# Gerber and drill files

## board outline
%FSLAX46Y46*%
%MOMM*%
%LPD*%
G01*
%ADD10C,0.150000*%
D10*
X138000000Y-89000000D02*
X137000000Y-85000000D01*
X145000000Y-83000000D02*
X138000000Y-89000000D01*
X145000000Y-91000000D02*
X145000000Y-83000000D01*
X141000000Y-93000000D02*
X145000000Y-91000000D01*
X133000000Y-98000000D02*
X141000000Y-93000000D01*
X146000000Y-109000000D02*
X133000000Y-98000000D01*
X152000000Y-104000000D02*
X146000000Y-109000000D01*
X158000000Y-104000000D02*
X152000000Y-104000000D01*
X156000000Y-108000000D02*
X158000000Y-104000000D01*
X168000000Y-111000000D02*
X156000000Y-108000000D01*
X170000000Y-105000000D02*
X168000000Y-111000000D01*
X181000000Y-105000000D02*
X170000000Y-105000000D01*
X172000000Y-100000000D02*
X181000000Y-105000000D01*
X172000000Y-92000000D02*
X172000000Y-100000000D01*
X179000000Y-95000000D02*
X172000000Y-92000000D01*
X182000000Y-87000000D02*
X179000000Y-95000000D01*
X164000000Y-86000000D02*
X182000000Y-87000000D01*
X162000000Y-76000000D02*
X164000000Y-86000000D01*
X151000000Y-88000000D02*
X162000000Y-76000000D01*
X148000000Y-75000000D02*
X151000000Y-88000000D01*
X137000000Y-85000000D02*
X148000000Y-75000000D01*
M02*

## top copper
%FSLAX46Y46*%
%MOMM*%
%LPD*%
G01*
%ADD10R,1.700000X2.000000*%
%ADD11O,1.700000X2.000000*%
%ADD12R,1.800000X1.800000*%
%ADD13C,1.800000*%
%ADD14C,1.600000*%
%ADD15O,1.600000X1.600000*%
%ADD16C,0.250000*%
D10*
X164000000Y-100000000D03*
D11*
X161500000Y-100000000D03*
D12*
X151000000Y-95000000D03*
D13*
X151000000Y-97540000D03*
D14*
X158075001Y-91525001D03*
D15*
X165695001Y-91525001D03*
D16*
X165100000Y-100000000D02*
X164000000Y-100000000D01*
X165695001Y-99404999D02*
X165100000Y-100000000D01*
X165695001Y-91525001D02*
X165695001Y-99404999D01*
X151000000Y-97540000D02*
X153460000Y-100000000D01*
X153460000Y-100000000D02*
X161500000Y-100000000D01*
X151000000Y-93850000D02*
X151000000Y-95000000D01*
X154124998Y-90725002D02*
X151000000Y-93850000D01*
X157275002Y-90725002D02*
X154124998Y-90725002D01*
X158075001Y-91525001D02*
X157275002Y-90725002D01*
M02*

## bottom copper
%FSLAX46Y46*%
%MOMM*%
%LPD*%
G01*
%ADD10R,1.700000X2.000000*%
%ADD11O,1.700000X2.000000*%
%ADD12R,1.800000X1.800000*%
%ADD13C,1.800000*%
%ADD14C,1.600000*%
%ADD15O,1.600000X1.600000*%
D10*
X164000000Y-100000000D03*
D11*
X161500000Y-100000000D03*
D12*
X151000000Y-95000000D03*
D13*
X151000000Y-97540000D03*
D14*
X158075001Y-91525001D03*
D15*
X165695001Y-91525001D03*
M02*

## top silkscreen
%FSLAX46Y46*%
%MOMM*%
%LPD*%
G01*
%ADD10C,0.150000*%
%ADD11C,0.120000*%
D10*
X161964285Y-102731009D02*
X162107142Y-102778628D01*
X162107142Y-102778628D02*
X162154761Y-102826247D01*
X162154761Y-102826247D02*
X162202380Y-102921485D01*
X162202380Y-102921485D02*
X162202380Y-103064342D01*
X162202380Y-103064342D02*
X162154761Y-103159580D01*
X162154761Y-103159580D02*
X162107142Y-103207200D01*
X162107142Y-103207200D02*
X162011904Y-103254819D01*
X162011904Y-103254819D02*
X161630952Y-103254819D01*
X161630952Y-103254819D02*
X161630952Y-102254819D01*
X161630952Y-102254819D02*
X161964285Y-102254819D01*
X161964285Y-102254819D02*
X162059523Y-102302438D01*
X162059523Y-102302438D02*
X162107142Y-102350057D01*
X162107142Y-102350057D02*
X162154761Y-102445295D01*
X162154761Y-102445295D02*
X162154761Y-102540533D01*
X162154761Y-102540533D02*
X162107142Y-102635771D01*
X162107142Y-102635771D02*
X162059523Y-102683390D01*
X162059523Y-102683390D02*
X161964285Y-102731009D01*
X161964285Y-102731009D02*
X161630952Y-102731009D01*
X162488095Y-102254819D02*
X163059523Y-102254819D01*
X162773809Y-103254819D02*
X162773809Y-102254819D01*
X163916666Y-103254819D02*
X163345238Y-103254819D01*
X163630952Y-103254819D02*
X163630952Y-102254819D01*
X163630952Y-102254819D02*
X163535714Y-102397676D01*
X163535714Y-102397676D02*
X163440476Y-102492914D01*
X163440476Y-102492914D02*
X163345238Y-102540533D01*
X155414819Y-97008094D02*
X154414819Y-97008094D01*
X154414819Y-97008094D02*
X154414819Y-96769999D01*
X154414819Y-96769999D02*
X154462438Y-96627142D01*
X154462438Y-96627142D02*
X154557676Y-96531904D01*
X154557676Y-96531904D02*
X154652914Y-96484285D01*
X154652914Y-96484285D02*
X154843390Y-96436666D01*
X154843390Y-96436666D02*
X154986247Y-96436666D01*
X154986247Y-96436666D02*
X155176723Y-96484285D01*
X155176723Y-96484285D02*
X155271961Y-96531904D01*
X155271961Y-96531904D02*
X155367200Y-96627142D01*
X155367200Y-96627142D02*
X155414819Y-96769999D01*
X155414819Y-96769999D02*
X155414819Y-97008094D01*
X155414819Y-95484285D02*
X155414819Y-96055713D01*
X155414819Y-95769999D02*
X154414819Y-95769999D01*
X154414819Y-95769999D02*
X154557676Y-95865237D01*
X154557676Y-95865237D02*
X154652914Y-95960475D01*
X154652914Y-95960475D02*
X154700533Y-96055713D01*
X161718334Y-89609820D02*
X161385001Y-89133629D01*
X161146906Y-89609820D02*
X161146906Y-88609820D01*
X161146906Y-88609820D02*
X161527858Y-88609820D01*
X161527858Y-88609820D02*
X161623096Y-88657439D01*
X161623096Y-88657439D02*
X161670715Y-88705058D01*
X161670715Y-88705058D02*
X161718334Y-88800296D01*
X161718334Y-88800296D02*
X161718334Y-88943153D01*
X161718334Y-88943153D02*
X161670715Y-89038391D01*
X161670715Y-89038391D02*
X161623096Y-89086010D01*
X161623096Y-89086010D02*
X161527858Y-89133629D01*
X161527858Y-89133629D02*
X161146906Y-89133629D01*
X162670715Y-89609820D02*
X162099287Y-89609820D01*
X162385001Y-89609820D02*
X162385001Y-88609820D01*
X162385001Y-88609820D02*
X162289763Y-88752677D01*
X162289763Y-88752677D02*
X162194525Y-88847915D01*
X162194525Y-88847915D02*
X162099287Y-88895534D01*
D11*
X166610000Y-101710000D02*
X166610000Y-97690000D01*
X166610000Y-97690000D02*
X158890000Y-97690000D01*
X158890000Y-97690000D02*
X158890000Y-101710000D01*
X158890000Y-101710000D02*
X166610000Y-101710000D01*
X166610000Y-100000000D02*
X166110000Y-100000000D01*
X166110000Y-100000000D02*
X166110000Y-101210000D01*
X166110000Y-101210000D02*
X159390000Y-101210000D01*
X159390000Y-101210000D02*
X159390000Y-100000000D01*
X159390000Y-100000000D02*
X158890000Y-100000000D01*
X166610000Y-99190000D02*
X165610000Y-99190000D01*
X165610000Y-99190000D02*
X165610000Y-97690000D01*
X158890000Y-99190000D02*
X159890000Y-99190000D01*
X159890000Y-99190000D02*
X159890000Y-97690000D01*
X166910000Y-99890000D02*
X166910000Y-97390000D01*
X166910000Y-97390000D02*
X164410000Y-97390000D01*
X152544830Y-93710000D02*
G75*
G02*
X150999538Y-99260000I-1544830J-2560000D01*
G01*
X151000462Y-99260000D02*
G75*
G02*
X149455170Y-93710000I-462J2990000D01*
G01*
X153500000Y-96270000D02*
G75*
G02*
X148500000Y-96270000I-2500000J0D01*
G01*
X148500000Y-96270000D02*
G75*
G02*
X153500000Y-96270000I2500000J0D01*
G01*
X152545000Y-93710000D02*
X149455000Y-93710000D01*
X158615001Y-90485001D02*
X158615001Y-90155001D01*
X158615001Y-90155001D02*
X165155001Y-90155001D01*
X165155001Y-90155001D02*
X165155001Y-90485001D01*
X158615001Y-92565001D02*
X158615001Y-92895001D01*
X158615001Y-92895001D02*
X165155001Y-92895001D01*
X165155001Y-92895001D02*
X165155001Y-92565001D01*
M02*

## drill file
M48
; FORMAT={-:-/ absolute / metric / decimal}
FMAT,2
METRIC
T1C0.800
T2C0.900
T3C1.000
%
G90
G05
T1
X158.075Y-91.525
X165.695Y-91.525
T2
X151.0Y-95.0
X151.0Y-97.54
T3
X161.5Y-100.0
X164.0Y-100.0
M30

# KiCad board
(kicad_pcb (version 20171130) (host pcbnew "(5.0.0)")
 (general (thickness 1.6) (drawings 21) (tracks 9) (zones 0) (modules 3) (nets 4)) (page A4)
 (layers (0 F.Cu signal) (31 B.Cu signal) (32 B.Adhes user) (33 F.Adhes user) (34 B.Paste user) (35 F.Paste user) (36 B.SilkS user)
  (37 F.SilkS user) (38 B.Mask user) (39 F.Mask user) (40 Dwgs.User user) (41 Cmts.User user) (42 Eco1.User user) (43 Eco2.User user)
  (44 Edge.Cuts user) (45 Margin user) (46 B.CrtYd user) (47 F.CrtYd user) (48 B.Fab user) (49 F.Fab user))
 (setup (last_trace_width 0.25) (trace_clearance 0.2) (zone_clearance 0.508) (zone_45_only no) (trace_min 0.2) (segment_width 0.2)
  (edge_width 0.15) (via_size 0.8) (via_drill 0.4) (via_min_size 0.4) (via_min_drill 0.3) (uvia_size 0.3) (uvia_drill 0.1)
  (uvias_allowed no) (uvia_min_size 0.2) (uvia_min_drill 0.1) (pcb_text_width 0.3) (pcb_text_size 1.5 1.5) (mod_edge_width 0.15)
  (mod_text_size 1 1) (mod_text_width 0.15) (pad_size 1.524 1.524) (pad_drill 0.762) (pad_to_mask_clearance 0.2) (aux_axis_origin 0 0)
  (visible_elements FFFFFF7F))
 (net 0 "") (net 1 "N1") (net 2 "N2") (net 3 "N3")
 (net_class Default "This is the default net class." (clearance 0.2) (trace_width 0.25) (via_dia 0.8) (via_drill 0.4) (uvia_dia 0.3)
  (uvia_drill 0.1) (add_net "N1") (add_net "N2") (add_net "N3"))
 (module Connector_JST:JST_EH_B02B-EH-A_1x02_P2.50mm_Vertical (layer F.Cu) (at 164 100 180)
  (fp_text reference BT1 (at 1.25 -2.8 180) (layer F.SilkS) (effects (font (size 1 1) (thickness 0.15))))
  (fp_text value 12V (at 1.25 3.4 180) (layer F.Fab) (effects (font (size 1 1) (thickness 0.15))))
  (fp_line (start -2.61 -1.71) (end -2.61 2.31) (layer F.SilkS) (width 0.12))
  (fp_line (start -2.61 2.31) (end 5.11 2.31) (layer F.SilkS) (width 0.12))
  (fp_line (start 5.11 2.31) (end 5.11 -1.71) (layer F.SilkS) (width 0.12))
  (fp_line (start 5.11 -1.71) (end -2.61 -1.71) (layer F.SilkS) (width 0.12))
  (fp_line (start -2.61 0) (end -2.11 0) (layer F.SilkS) (width 0.12))
  (fp_line (start -2.11 0) (end -2.11 -1.21) (layer F.SilkS) (width 0.12))
  (fp_line (start -2.11 -1.21) (end 4.61 -1.21) (layer F.SilkS) (width 0.12))
  (fp_line (start 4.61 -1.21) (end 4.61 0) (layer F.SilkS) (width 0.12))
  (fp_line (start 4.61 0) (end 5.11 0) (layer F.SilkS) (width 0.12))
  (fp_line (start -2.61 0.81) (end -1.61 0.81) (layer F.SilkS) (width 0.12))
  (fp_line (start -1.61 0.81) (end -1.61 2.31) (layer F.SilkS) (width 0.12))
  (fp_line (start 5.11 0.81) (end 4.11 0.81) (layer F.SilkS) (width 0.12))
  (fp_line (start 4.11 0.81) (end 4.11 2.31) (layer F.SilkS) (width 0.12))
  (fp_line (start -2.91 0.11) (end -2.91 2.61) (layer F.SilkS) (width 0.12))
  (fp_line (start -2.91 2.61) (end -0.41 2.61) (layer F.SilkS) (width 0.12))
  (pad 1 thru_hole rect (at 0 0 180) (size 1.7 2) (drill 1) (layers *.Cu *.Mask) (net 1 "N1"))
  (pad 2 thru_hole oval (at 2.5 0 180) (size 1.7 2) (drill 1) (layers *.Cu *.Mask) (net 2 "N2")))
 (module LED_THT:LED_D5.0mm (layer F.Cu) (at 151 95 270)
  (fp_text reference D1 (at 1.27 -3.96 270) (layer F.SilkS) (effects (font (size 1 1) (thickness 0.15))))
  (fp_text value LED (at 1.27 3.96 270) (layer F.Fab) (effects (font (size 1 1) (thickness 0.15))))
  (fp_arc (start 1.27 0) (end -1.29 -1.54483) (angle 148.9) (layer F.SilkS) (width 0.12))
  (fp_arc (start 1.27 0) (end -1.29 1.54483) (angle -148.9) (layer F.SilkS) (width 0.12))
  (fp_circle (center 1.27 0) (end 3.77 0) (layer F.SilkS) (width 0.12))
  (fp_line (start -1.29 -1.545) (end -1.29 1.545) (layer F.SilkS) (width 0.12))
  (pad 1 thru_hole rect (at 0 0 270) (size 1.8 1.8) (drill 0.9) (layers *.Cu *.Mask) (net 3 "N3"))
  (pad 2 thru_hole circle (at 2.54 0 270) (size 1.8 1.8) (drill 0.9) (layers *.Cu *.Mask) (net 2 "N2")))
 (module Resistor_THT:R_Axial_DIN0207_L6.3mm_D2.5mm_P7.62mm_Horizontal (layer F.Cu) (at 158.075001 91.525001)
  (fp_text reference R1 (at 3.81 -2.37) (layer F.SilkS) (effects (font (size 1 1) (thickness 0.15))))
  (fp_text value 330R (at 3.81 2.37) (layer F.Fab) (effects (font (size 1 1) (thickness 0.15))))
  (fp_line (start 0.54 -1.04) (end 0.54 -1.37) (layer F.SilkS) (width 0.12))
  (fp_line (start 0.54 -1.37) (end 7.08 -1.37) (layer F.SilkS) (width 0.12))
  (fp_line (start 7.08 -1.37) (end 7.08 -1.04) (layer F.SilkS) (width 0.12))
  (fp_line (start 0.54 1.04) (end 0.54 1.37) (layer F.SilkS) (width 0.12))
  (fp_line (start 0.54 1.37) (end 7.08 1.37) (layer F.SilkS) (width 0.12))
  (fp_line (start 7.08 1.37) (end 7.08 1.04) (layer F.SilkS) (width 0.12))
  (pad 1 thru_hole circle (at 0 0) (size 1.6 1.6) (drill 0.8) (layers *.Cu *.Mask) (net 3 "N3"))
  (pad 2 thru_hole oval (at 7.62 0) (size 1.6 1.6) (drill 0.8) (layers *.Cu *.Mask) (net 1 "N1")))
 (gr_line (start 138 89) (end 137 85) (layer Edge.Cuts) (width 0.15))
 (gr_line (start 145 83) (end 138 89) (layer Edge.Cuts) (width 0.15))
 (gr_line (start 145 91) (end 145 83) (layer Edge.Cuts) (width 0.15))
 (gr_line (start 141 93) (end 145 91) (layer Edge.Cuts) (width 0.15))
 (gr_line (start 133 98) (end 141 93) (layer Edge.Cuts) (width 0.15))
 (gr_line (start 146 109) (end 133 98) (layer Edge.Cuts) (width 0.15))
 (gr_line (start 152 104) (end 146 109) (layer Edge.Cuts) (width 0.15))
 (gr_line (start 158 104) (end 152 104) (layer Edge.Cuts) (width 0.15))
 (gr_line (start 156 108) (end 158 104) (layer Edge.Cuts) (width 0.15))
 (gr_line (start 168 111) (end 156 108) (layer Edge.Cuts) (width 0.15))
 (gr_line (start 170 105) (end 168 111) (layer Edge.Cuts) (width 0.15))
 (gr_line (start 181 105) (end 170 105) (layer Edge.Cuts) (width 0.15))
 (gr_line (start 172 100) (end 181 105) (layer Edge.Cuts) (width 0.15))
 (gr_line (start 172 92) (end 172 100) (layer Edge.Cuts) (width 0.15))
 (gr_line (start 179 95) (end 172 92) (layer Edge.Cuts) (width 0.15))
 (gr_line (start 182 87) (end 179 95) (layer Edge.Cuts) (width 0.15))
 (gr_line (start 164 86) (end 182 87) (layer Edge.Cuts) (width 0.15))
 (gr_line (start 162 76) (end 164 86) (layer Edge.Cuts) (width 0.15))
 (gr_line (start 151 88) (end 162 76) (layer Edge.Cuts) (width 0.15))
 (gr_line (start 148 75) (end 151 88) (layer Edge.Cuts) (width 0.15))
 (gr_line (start 137 85) (end 148 75) (layer Edge.Cuts) (width 0.15))
 (segment (start 165.1 100) (end 164 100) (width 0.25) (layer F.Cu) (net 1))
 (segment (start 165.695001 99.404999) (end 165.1 100) (width 0.25) (layer F.Cu) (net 1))
 (segment (start 165.695001 91.525001) (end 165.695001 99.404999) (width 0.25) (layer F.Cu) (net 1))
 (segment (start 151 97.54) (end 153.46 100) (width 0.25) (layer F.Cu) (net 2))
 (segment (start 153.46 100) (end 161.5 100) (width 0.25) (layer F.Cu) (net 2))
 (segment (start 151 93.85) (end 151 95) (width 0.25) (layer F.Cu) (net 3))
 (segment (start 154.124998 90.725002) (end 151 93.85) (width 0.25) (layer F.Cu) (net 3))
 (segment (start 157.275002 90.725002) (end 154.124998 90.725002) (width 0.25) (layer F.Cu) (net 3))
 (segment (start 158.075001 91.525001) (end 157.275002 90.725002) (width 0.25) (layer F.Cu) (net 3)))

